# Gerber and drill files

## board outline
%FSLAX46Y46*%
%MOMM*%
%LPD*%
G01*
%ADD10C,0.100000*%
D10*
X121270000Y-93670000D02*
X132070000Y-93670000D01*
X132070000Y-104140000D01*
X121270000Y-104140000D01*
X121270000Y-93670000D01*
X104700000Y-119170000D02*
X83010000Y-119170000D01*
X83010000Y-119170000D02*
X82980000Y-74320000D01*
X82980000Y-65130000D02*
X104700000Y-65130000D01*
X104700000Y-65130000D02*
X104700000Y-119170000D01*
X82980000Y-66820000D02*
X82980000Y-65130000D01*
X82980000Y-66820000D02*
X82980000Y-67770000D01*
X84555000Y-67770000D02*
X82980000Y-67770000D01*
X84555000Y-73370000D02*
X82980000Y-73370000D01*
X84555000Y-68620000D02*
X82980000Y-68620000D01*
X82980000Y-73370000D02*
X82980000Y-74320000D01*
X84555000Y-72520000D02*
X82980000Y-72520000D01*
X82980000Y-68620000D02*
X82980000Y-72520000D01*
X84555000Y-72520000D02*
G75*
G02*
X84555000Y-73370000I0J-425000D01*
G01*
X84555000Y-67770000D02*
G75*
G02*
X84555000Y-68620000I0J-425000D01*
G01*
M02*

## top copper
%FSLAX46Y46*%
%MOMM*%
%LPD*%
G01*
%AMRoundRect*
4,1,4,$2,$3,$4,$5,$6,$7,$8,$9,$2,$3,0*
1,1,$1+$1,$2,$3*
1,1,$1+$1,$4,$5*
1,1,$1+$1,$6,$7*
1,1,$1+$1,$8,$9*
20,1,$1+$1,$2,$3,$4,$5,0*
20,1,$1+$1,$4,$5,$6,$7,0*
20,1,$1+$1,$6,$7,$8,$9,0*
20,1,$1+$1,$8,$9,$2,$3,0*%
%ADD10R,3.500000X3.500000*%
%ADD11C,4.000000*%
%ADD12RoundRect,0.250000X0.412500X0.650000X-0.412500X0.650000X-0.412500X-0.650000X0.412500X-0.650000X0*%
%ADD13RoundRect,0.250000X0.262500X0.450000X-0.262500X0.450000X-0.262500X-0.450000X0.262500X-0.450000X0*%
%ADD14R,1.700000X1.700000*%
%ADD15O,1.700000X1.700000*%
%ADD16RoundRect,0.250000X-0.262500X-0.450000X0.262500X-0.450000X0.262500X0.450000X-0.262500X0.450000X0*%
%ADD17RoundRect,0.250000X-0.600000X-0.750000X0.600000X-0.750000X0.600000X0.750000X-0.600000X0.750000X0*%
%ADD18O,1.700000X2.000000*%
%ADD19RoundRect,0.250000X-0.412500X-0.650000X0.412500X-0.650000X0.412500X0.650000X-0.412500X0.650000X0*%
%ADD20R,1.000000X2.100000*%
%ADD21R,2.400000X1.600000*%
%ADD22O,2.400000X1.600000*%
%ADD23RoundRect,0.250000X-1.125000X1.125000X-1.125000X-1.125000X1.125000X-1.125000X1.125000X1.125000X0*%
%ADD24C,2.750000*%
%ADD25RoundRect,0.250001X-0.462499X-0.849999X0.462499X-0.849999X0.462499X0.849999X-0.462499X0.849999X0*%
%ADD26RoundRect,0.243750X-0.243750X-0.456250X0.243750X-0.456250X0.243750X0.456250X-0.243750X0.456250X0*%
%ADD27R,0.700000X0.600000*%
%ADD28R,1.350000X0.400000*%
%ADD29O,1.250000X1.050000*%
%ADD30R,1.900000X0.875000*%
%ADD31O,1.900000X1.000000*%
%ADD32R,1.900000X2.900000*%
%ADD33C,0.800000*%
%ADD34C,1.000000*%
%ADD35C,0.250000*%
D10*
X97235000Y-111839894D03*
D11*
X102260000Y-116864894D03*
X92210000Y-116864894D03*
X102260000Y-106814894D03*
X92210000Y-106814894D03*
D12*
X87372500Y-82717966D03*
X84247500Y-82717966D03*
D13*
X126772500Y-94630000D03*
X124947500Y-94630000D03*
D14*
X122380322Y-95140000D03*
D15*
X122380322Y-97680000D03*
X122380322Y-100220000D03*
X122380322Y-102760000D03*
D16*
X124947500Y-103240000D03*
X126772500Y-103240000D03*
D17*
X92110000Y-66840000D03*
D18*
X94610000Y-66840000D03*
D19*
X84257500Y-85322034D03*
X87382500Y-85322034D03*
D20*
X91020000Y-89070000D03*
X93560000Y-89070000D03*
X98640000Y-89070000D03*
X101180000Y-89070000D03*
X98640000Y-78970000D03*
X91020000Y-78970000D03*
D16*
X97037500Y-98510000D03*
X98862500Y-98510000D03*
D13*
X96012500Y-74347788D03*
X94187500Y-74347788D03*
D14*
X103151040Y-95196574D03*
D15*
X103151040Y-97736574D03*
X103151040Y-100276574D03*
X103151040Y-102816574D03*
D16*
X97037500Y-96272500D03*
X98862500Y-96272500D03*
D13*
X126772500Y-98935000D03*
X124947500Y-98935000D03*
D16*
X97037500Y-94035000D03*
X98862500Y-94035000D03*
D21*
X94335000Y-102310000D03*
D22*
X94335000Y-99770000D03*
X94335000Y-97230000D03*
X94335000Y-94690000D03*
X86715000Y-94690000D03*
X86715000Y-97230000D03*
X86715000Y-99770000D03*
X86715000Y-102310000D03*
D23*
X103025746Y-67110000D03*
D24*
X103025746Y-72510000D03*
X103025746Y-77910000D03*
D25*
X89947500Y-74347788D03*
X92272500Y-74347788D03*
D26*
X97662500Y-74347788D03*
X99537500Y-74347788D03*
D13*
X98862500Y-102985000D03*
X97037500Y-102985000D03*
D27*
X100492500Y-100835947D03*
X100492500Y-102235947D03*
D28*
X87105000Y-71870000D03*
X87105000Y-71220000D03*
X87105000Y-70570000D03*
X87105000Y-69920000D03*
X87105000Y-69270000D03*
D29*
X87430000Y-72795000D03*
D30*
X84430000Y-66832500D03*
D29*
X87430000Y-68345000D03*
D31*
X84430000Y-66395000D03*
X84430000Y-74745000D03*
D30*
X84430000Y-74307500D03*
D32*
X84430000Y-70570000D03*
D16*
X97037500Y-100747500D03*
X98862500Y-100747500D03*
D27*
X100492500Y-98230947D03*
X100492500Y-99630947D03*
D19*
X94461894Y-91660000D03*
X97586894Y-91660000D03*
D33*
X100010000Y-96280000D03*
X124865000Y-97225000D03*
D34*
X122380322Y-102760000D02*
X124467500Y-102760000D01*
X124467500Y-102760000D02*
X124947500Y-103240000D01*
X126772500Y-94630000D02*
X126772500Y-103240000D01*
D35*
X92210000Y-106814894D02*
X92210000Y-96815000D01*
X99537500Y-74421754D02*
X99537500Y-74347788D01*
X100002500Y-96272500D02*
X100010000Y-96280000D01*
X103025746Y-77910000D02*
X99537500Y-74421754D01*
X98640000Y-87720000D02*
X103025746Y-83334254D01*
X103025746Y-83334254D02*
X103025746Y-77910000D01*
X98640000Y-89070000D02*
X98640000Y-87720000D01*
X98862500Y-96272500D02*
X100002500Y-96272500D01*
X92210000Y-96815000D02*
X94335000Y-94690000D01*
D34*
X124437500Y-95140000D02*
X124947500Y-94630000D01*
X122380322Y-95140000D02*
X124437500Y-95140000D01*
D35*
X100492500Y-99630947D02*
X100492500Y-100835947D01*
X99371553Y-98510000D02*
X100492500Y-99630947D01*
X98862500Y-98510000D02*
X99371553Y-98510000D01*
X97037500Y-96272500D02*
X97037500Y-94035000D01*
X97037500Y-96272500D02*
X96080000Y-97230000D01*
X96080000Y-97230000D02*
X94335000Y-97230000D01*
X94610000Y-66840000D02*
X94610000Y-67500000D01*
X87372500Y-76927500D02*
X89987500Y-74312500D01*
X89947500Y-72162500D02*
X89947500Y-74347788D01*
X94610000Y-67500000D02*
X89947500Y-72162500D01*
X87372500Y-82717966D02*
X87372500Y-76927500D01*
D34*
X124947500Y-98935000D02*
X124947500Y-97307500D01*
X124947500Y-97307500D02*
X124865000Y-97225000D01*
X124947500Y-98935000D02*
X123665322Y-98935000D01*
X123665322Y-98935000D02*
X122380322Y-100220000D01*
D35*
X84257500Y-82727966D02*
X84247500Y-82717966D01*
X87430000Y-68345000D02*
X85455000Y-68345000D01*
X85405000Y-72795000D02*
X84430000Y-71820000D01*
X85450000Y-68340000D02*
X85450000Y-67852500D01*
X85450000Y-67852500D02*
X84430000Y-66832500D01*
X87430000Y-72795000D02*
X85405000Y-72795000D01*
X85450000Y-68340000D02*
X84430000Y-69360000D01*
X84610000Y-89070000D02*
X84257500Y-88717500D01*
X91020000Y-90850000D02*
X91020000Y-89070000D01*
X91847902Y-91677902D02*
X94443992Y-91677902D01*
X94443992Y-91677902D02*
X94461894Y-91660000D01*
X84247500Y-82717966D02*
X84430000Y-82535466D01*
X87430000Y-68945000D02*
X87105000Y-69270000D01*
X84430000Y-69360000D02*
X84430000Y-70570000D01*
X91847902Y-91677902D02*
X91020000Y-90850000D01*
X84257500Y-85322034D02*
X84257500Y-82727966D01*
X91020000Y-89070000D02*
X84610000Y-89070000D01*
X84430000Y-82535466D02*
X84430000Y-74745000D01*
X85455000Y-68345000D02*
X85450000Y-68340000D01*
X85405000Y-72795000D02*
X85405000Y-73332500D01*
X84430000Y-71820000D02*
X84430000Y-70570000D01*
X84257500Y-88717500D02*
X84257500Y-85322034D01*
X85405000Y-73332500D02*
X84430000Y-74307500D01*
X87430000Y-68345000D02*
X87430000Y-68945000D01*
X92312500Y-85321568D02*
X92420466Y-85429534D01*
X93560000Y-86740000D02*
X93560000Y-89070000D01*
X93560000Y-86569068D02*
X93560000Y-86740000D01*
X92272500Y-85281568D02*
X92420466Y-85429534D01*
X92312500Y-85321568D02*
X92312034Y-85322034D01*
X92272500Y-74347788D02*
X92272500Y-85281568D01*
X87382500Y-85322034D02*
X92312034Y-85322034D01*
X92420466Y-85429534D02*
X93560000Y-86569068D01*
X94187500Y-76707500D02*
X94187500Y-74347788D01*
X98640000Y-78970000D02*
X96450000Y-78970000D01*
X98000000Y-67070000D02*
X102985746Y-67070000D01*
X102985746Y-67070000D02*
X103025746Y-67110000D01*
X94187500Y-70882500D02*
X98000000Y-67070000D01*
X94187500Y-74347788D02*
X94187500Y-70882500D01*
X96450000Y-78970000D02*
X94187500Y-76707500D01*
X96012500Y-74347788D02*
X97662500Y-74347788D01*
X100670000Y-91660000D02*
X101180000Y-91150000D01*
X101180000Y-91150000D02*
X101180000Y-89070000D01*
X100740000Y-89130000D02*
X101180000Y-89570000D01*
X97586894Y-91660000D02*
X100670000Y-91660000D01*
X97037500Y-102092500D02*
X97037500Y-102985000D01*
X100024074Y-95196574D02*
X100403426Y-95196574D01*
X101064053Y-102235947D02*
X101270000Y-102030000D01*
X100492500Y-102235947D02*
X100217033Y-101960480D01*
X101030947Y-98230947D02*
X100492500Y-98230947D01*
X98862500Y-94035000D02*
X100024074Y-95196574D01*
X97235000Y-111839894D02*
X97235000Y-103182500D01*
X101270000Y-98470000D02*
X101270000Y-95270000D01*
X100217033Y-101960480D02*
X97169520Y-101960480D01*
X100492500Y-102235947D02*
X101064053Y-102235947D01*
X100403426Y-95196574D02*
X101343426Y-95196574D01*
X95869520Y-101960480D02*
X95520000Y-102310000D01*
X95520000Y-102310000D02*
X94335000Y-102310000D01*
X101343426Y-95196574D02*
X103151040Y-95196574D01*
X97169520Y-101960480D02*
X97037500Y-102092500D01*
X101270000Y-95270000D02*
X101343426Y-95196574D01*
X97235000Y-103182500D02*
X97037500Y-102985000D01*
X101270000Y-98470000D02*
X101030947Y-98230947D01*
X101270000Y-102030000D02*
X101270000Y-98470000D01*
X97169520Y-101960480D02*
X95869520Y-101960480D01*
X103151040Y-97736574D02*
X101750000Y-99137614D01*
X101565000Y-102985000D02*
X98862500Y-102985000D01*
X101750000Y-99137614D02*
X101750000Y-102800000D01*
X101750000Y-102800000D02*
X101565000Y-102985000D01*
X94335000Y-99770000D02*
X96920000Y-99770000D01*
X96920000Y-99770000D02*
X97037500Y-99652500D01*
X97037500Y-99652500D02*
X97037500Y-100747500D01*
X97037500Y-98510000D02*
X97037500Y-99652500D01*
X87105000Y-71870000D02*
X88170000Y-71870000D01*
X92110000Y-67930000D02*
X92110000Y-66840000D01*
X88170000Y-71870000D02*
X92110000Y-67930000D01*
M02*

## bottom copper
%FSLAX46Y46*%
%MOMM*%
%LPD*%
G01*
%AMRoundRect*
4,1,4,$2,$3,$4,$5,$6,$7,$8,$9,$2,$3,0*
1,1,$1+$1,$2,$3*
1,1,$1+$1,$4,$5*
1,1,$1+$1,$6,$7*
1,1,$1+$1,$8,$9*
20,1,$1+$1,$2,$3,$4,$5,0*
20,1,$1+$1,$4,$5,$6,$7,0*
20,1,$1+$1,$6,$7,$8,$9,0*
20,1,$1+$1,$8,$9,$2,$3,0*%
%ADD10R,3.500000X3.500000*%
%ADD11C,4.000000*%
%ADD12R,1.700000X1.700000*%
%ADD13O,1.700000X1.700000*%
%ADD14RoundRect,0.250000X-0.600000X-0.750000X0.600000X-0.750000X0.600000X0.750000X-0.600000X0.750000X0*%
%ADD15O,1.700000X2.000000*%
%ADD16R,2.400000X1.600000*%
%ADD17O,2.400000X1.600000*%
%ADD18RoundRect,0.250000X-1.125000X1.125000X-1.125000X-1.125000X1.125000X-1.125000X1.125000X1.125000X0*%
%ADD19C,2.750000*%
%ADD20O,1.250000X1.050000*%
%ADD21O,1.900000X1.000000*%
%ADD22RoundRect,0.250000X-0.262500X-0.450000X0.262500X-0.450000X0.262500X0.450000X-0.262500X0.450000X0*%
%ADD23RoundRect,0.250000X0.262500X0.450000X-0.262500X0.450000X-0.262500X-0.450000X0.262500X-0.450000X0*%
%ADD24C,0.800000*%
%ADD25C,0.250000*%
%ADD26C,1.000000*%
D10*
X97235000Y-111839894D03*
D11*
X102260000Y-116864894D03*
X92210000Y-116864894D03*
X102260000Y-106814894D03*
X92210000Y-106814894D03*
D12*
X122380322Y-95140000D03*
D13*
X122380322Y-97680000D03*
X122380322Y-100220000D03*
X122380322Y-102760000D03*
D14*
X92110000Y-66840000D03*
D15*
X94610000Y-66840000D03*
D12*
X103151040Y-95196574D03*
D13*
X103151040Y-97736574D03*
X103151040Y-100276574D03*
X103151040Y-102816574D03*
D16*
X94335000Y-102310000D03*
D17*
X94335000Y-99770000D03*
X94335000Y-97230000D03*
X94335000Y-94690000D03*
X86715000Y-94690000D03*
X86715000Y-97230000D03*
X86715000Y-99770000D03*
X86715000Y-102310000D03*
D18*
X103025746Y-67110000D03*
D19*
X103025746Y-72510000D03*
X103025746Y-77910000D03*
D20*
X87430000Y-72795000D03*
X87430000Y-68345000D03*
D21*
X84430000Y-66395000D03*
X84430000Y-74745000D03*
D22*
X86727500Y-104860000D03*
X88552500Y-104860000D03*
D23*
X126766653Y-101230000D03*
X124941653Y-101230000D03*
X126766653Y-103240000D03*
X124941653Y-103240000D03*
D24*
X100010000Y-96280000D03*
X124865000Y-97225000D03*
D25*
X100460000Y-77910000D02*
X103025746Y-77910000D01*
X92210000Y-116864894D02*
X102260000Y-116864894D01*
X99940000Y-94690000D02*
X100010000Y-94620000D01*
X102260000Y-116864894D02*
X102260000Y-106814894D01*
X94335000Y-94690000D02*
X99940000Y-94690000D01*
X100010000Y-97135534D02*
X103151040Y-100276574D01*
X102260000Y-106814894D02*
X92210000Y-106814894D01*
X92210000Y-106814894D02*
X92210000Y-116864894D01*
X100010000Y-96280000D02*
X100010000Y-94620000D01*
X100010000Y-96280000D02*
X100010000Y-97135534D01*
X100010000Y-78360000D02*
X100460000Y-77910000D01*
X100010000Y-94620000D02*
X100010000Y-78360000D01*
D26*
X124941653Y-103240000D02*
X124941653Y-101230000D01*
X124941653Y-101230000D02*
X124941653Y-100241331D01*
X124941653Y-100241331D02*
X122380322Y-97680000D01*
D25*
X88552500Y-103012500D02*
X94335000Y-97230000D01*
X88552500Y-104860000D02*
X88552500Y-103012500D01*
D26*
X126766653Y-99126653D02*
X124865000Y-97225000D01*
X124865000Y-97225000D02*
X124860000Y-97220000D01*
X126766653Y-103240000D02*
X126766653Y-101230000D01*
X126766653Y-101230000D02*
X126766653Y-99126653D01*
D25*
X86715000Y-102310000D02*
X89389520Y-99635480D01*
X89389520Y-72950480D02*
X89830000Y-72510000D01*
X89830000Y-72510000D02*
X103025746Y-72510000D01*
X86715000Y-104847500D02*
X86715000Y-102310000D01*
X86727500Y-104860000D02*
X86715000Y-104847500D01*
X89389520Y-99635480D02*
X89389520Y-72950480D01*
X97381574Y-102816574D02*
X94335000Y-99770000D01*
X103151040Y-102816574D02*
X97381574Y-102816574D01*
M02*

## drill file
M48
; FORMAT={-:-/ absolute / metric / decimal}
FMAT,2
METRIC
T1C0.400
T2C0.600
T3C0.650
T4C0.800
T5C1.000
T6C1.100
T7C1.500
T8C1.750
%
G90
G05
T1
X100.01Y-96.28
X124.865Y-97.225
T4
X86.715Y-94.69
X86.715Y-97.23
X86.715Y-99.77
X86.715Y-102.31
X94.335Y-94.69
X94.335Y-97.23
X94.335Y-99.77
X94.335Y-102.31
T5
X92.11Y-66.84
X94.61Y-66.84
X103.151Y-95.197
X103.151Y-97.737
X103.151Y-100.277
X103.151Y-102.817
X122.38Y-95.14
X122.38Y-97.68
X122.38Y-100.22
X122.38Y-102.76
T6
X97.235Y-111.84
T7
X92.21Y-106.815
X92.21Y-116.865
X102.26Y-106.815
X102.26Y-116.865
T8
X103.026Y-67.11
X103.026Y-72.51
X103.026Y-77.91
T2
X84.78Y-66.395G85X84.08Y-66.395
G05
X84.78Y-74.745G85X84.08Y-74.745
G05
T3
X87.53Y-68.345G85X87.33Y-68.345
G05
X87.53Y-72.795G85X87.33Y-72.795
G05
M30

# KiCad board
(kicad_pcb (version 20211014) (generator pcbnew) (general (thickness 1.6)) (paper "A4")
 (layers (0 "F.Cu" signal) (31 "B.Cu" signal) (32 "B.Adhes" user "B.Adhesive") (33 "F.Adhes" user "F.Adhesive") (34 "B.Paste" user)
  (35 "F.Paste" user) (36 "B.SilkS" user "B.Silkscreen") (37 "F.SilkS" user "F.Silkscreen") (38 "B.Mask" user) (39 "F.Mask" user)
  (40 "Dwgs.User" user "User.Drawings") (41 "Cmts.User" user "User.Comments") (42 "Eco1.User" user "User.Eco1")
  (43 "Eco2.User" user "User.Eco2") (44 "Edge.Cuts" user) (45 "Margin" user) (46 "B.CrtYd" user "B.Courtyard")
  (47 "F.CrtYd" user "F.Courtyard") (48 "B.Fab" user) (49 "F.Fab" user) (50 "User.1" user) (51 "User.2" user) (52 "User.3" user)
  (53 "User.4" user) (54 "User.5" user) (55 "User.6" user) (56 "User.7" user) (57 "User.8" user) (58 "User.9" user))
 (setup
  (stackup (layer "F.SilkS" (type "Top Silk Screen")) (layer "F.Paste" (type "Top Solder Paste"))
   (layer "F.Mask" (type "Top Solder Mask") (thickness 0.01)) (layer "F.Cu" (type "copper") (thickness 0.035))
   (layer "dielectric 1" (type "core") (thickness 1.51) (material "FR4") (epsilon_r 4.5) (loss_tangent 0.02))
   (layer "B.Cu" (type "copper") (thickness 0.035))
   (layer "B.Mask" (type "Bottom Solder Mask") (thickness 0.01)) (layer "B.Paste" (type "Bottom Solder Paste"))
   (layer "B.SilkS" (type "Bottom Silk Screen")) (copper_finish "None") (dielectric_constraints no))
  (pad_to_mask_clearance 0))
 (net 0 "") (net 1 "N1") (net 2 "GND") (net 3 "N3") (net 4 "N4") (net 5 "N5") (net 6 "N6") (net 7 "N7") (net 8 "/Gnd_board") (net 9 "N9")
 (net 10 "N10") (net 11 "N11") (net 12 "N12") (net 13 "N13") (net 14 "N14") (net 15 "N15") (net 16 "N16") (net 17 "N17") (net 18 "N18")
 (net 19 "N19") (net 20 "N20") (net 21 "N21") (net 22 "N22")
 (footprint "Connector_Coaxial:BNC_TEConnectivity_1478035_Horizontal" (layer "F.Cu") (at 97.235 111.839894 -90)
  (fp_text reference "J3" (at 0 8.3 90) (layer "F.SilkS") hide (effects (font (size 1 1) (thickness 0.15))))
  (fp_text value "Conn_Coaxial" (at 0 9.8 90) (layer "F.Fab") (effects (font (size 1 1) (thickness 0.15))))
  (pad "1" thru_hole rect (at 0 0 270) (size 3.5 3.5) (drill 1.1) (layers *.Cu *.Mask) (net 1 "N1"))
  (pad "2" thru_hole circle (at 5.025 -5.025 270) (size 4 4) (drill 1.5) (layers *.Cu *.Mask) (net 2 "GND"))
  (pad "2" thru_hole circle (at 5.025 5.025 270) (size 4 4) (drill 1.5) (layers *.Cu *.Mask) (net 2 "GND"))
  (pad "2" thru_hole circle (at -5.025 -5.025 270) (size 4 4) (drill 1.5) (layers *.Cu *.Mask) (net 2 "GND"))
  (pad "2" thru_hole circle (at -5.025 5.025 270) (size 4 4) (drill 1.5) (layers *.Cu *.Mask) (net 2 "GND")))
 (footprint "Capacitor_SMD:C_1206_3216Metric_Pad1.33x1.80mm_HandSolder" (layer "F.Cu") (at 85.81 82.717966 180)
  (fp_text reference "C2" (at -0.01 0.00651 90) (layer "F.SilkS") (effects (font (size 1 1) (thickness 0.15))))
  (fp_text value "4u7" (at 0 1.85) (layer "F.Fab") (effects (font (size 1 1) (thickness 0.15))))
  (pad "1" smd roundrect locked (at -1.5625 0 180) (size 1.325 1.8) (layers "F.Cu" "F.Paste" "F.Mask") (roundrect_rratio 0.188679)
   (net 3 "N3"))
  (pad "2" smd roundrect locked (at 1.5625 0 180) (size 1.325 1.8) (layers "F.Cu" "F.Paste" "F.Mask") (roundrect_rratio 0.188679)
   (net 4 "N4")))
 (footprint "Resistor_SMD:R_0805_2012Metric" (layer "F.Cu") (at 125.86 94.63 180)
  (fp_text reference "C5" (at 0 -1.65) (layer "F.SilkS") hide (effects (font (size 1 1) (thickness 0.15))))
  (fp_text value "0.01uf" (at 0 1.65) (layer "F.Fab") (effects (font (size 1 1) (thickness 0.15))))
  (pad "1" smd roundrect locked (at -0.9125 0 180) (size 1.025 1.4) (layers "F.Cu" "F.Paste" "F.Mask") (roundrect_rratio 0.243902)
   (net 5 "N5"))
  (pad "2" smd roundrect locked (at 0.9125 0 180) (size 1.025 1.4) (layers "F.Cu" "F.Paste" "F.Mask") (roundrect_rratio 0.243902)
   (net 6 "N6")))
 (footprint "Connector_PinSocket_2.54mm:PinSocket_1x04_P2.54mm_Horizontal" (layer "F.Cu") (at 122.380322 95.14)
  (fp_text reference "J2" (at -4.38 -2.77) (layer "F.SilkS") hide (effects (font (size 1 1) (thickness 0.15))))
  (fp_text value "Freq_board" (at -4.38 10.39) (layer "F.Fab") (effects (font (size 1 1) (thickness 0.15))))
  (pad "1" thru_hole rect locked (at 0 0) (size 1.7 1.7) (drill 1) (layers *.Cu *.Mask) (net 6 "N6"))
  (pad "2" thru_hole oval locked (at 0 2.54) (size 1.7 1.7) (drill 1) (layers *.Cu *.Mask) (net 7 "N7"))
  (pad "3" thru_hole oval locked (at 0 5.08) (size 1.7 1.7) (drill 1) (layers *.Cu *.Mask) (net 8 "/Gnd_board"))
  (pad "4" thru_hole oval locked (at 0 7.62) (size 1.7 1.7) (drill 1) (layers *.Cu *.Mask) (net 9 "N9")))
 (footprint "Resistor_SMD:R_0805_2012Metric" (layer "F.Cu") (at 125.86 103.24)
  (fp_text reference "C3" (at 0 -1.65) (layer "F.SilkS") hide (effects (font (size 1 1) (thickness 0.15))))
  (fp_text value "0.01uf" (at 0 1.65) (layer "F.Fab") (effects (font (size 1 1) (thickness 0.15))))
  (pad "1" smd roundrect locked (at -0.9125 0) (size 1.025 1.4) (layers "F.Cu" "F.Paste" "F.Mask") (roundrect_rratio 0.243902) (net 9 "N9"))
  (pad "2" smd roundrect locked (at 0.9125 0) (size 1.025 1.4) (layers "F.Cu" "F.Paste" "F.Mask") (roundrect_rratio 0.243902) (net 5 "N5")))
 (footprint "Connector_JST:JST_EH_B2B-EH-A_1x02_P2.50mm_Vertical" (layer "F.Cu") (at 92.11 66.84)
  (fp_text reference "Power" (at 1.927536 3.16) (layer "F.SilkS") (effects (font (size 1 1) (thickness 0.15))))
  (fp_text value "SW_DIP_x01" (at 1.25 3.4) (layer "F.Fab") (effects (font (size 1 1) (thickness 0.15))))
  (pad "1" thru_hole roundrect locked (at 0 0) (size 1.7 2) (drill 1) (layers *.Cu *.Mask) (roundrect_rratio 0.147059) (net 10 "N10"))
  (pad "2" thru_hole oval locked (at 2.5 0) (size 1.7 2) (drill 1) (layers *.Cu *.Mask) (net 3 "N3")))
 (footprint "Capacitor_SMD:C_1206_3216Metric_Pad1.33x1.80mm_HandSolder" (layer "F.Cu") (at 85.82 85.322034)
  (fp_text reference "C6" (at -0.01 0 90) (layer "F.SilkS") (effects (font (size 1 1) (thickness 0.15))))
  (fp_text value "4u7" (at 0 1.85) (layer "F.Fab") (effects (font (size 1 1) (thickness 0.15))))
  (pad "1" smd roundrect locked (at -1.5625 0) (size 1.325 1.8) (layers "F.Cu" "F.Paste" "F.Mask") (roundrect_rratio 0.188679) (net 4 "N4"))
  (pad "2" smd roundrect locked (at 1.5625 0) (size 1.325 1.8) (layers "F.Cu" "F.Paste" "F.Mask") (roundrect_rratio 0.188679) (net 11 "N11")))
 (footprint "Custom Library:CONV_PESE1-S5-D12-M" (layer "F.Cu") (at 96.1 84.02 90)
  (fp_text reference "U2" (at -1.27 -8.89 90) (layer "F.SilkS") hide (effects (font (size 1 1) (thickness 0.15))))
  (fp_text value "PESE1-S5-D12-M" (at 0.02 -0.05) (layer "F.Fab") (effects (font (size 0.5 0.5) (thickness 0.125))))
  (pad "1" smd rect (at -5.05 -5.08 90) (size 2.1 1) (layers "F.Cu" "F.Paste" "F.Mask") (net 4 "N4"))
  (pad "2" smd rect (at -5.05 -2.54 90) (size 2.1 1) (layers "F.Cu" "F.Paste" "F.Mask") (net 11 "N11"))
  (pad "4" smd rect (at -5.05 2.54 90) (size 2.1 1) (layers "F.Cu" "F.Paste" "F.Mask") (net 2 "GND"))
  (pad "5" smd rect (at -5.05 5.08 90) (size 2.1 1) (layers "F.Cu" "F.Paste" "F.Mask") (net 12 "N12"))
  (pad "7" smd rect (at 5.05 2.54 90) (size 2.1 1) (layers "F.Cu" "F.Paste" "F.Mask") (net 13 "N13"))
  (pad "10" smd rect (at 5.05 -5.08 90) (size 2.1 1) (layers "F.Cu" "F.Paste" "F.Mask")))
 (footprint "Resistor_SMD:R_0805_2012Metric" (layer "F.Cu") (at 97.95 98.51)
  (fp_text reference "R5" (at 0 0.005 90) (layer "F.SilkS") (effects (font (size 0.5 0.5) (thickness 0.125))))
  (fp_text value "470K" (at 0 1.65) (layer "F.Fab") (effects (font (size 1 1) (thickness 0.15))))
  (pad "1" smd roundrect locked (at -0.9125 0) (size 1.025 1.4) (layers "F.Cu" "F.Paste" "F.Mask") (roundrect_rratio 0.243902)
   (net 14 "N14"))
  (pad "2" smd roundrect locked (at 0.9125 0) (size 1.025 1.4) (layers "F.Cu" "F.Paste" "F.Mask") (roundrect_rratio 0.243902) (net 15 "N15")))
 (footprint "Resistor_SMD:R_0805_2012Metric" (layer "F.Cu") (at 95.1 74.347788 180)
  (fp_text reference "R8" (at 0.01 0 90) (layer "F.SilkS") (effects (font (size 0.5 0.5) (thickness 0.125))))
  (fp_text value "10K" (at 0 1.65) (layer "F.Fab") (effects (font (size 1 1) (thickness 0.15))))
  (pad "1" smd roundrect locked (at -0.9125 0 180) (size 1.025 1.4) (layers "F.Cu" "F.Paste" "F.Mask") (roundrect_rratio 0.243902)
   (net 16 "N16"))
  (pad "2" smd roundrect locked (at 0.9125 0 180) (size 1.025 1.4) (layers "F.Cu" "F.Paste" "F.Mask") (roundrect_rratio 0.243902)
   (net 13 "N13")))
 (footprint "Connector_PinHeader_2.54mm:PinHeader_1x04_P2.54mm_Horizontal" (layer "F.Cu") (at 103.15104 95.196574)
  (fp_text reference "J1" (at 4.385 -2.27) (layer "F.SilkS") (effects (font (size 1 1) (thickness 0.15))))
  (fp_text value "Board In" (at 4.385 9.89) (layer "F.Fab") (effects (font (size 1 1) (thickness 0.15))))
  (pad "1" thru_hole rect locked (at 0 0) (size 1.7 1.7) (drill 1) (layers *.Cu *.Mask) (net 1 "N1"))
  (pad "2" thru_hole oval locked (at 0 2.54) (size 1.7 1.7) (drill 1) (layers *.Cu *.Mask) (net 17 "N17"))
  (pad "3" thru_hole oval locked (at 0 5.08) (size 1.7 1.7) (drill 1) (layers *.Cu *.Mask) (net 2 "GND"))
  (pad "4" thru_hole oval locked (at 0 7.62) (size 1.7 1.7) (drill 1) (layers *.Cu *.Mask) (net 14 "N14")))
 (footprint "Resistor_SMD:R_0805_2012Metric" (layer "F.Cu") (at 97.95 96.2725)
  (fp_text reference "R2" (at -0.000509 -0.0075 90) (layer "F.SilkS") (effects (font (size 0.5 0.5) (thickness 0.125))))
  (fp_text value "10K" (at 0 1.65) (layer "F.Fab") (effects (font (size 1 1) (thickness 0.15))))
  (pad "1" smd roundrect locked (at -0.9125 0) (size 1.025 1.4) (layers "F.Cu" "F.Paste" "F.Mask") (roundrect_rratio 0.243902)
   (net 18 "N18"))
  (pad "2" smd roundrect locked (at 0.9125 0) (size 1.025 1.4) (layers "F.Cu" "F.Paste" "F.Mask") (roundrect_rratio 0.243902) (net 2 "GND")))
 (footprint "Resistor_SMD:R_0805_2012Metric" (layer "F.Cu") (at 125.86 98.935 180)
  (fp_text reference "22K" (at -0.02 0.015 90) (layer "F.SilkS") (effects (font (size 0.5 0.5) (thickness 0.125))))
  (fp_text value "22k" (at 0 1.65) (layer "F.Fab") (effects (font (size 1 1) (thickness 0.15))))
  (pad "1" smd roundrect locked (at -0.9125 0 180) (size 1.025 1.4) (layers "F.Cu" "F.Paste" "F.Mask") (roundrect_rratio 0.243902)
   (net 5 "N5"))
  (pad "2" smd roundrect locked (at 0.9125 0 180) (size 1.025 1.4) (layers "F.Cu" "F.Paste" "F.Mask") (roundrect_rratio 0.243902)
   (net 8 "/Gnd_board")))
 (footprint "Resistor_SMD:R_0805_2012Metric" (layer "F.Cu") (at 97.95 94.035)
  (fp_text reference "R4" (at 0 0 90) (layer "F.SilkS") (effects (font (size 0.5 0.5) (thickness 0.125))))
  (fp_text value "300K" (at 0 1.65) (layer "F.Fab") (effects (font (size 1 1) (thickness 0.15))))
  (pad "1" smd roundrect locked (at -0.9125 0) (size 1.025 1.4) (layers "F.Cu" "F.Paste" "F.Mask") (roundrect_rratio 0.243902)
   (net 18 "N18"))
  (pad "2" smd roundrect locked (at 0.9125 0) (size 1.025 1.4) (layers "F.Cu" "F.Paste" "F.Mask") (roundrect_rratio 0.243902) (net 1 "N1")))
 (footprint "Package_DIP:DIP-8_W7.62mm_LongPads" (layer "F.Cu") (at 94.335 102.31 180)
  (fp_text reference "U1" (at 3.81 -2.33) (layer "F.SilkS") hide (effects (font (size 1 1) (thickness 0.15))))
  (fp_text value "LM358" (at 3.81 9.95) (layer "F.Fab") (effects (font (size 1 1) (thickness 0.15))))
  (pad "1" thru_hole rect locked (at 0 0 180) (size 2.4 1.6) (drill 0.8) (layers *.Cu *.Mask) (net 1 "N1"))
  (pad "2" thru_hole oval locked (at 0 2.54 180) (size 2.4 1.6) (drill 0.8) (layers *.Cu *.Mask) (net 14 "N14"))
  (pad "3" thru_hole oval locked (at 0 5.08 180) (size 2.4 1.6) (drill 0.8) (layers *.Cu *.Mask) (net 18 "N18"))
  (pad "4" thru_hole oval locked (at 0 7.62 180) (size 2.4 1.6) (drill 0.8) (layers *.Cu *.Mask) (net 2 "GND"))
  (pad "5" thru_hole oval locked (at 7.62 7.62 180) (size 2.4 1.6) (drill 0.8) (layers *.Cu *.Mask))
  (pad "6" thru_hole oval locked (at 7.62 5.08 180) (size 2.4 1.6) (drill 0.8) (layers *.Cu *.Mask))
  (pad "7" thru_hole oval locked (at 7.62 2.54 180) (size 2.4 1.6) (drill 0.8) (layers *.Cu *.Mask))
  (pad "8" thru_hole oval locked (at 7.62 0 180) (size 2.4 1.6) (drill 0.8) (layers *.Cu *.Mask) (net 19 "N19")))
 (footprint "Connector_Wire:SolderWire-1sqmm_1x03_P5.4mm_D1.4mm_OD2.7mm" (layer "F.Cu") (at 103.025746 67.11 -90)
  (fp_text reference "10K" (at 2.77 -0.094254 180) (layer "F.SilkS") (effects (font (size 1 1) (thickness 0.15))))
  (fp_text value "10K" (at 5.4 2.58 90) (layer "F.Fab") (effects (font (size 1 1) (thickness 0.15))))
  (pad "1" thru_hole roundrect locked (at 0 0 270) (size 2.75 2.75) (drill 1.75) (layers *.Cu *.Mask) (roundrect_rratio 0.090909)
   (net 13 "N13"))
  (pad "2" thru_hole circle locked (at 5.4 0 270) (size 2.75 2.75) (drill 1.75) (layers *.Cu *.Mask) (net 19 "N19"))
  (pad "3" thru_hole circle locked (at 10.8 0 270) (size 2.75 2.75) (drill 1.75) (layers *.Cu *.Mask) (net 2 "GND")))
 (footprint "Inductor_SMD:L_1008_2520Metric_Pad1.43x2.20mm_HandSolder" (layer "F.Cu") (at 91.11 74.347788)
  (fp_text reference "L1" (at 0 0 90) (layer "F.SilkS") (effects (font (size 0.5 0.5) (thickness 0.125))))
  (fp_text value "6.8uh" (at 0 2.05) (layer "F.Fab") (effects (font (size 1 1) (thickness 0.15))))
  (pad "1" smd roundrect locked (at -1.1625 0) (size 1.425 2.2) (layers "F.Cu" "F.Paste" "F.Mask") (roundrect_rratio 0.175439) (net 3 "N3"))
  (pad "2" smd roundrect locked (at 1.1625 0) (size 1.425 2.2) (layers "F.Cu" "F.Paste" "F.Mask") (roundrect_rratio 0.175439) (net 11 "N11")))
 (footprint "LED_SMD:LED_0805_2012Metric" (layer "F.Cu") (at 98.6 74.347788)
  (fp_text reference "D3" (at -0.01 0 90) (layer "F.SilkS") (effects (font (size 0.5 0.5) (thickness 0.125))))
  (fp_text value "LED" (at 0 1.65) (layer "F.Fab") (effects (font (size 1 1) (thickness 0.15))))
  (pad "1" smd roundrect locked (at -0.9375 0) (size 0.975 1.4) (layers "F.Cu" "F.Paste" "F.Mask") (roundrect_rratio 0.25) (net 16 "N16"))
  (pad "2" smd roundrect locked (at 0.9375 0) (size 0.975 1.4) (layers "F.Cu" "F.Paste" "F.Mask") (roundrect_rratio 0.25) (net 2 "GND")))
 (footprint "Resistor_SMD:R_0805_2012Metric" (layer "F.Cu") (at 97.95 102.985 180)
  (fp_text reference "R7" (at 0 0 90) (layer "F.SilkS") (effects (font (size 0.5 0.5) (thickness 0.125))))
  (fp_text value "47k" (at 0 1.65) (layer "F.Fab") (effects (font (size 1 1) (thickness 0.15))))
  (pad "1" smd roundrect locked (at -0.9125 0 180) (size 1.025 1.4) (layers "F.Cu" "F.Paste" "F.Mask") (roundrect_rratio 0.243902)
   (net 17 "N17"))
  (pad "2" smd roundrect locked (at 0.9125 0 180) (size 1.025 1.4) (layers "F.Cu" "F.Paste" "F.Mask") (roundrect_rratio 0.243902)
   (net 1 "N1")))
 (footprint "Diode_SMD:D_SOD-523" (layer "F.Cu") (at 100.4925 101.535947 -90)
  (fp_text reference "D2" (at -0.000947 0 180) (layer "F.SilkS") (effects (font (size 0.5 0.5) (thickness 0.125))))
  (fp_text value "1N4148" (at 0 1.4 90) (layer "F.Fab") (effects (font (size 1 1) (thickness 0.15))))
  (pad "1" smd rect locked (at -0.7 0 90) (size 0.6 0.7) (layers "F.Cu" "F.Paste" "F.Mask") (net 15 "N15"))
  (pad "2" smd rect locked (at 0.7 0 90) (size 0.6 0.7) (layers "F.Cu" "F.Paste" "F.Mask") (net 1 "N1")))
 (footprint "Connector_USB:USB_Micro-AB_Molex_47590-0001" (layer "F.Cu") (at 84.43 70.57 -90)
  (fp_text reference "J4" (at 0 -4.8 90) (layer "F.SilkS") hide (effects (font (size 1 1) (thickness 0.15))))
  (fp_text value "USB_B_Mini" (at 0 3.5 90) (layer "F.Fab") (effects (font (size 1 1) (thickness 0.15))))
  (fp_line (start -3.75 1.45) (end -2.8 1.45) (layer "Edge.Cuts") (width 0.1))
  (fp_line (start -2.8 -0.125) (end -2.8 1.45) (layer "Edge.Cuts") (width 0.1))
  (fp_line (start 2.8 -0.125) (end 2.8 1.45) (layer "Edge.Cuts") (width 0.1))
  (fp_line (start -1.95 -0.125) (end -1.95 1.45) (layer "Edge.Cuts") (width 0.1))
  (fp_line (start 2.8 1.45) (end 3.75 1.45) (layer "Edge.Cuts") (width 0.1))
  (fp_line (start 1.95 -0.125) (end 1.95 1.45) (layer "Edge.Cuts") (width 0.1))
  (fp_line (start -1.95 1.45) (end 1.95 1.45) (layer "Edge.Cuts") (width 0.1))
  (fp_arc (start 1.95 -0.125) (mid 2.375 -0.55) (end 2.8 -0.125) (layer "Edge.Cuts") (width 0.1))
  (fp_arc (start -2.8 -0.125) (mid -2.375 -0.55) (end -1.95 -0.125) (layer "Edge.Cuts") (width 0.1))
  (pad "" smd rect locked (at -3.5 0 270) (size 0.3 0.85) (layers "F.Paste"))
  (pad "" smd rect locked (at 3.5 0 270) (size 0.3 0.85) (layers "F.Paste"))
  (pad "1" smd rect locked (at 1.3 -2.675 270) (size 0.4 1.35) (layers "F.Cu" "F.Paste" "F.Mask") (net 10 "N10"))
  (pad "2" smd rect locked (at 0.65 -2.675 270) (size 0.4 1.35) (layers "F.Cu" "F.Paste" "F.Mask") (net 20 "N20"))
  (pad "3" smd rect locked (at 0 -2.675 270) (size 0.4 1.35) (layers "F.Cu" "F.Paste" "F.Mask") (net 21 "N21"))
  (pad "4" smd rect locked (at -0.65 -2.675 270) (size 0.4 1.35) (layers "F.Cu" "F.Paste" "F.Mask") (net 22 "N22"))
  (pad "5" smd rect locked (at -1.3 -2.675 270) (size 0.4 1.35) (layers "F.Cu" "F.Paste" "F.Mask") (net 4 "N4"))
  (pad "6" thru_hole oval locked (at 2.225 -3 270) (size 1.05 1.25) (drill oval 0.65 0.85) (layers *.Cu *.Mask) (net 4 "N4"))
  (pad "6" smd rect locked (at -3.7375 0 270) (size 0.875 1.9) (layers "F.Cu" "F.Mask") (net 4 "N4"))
  (pad "6" thru_hole oval locked (at -2.225 -3 270) (size 1.05 1.25) (drill oval 0.65 0.85) (layers *.Cu *.Mask) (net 4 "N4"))
  (pad "6" thru_hole oval locked (at -4.175 0 270) (size 1 1.9) (drill oval 0.6 1.3) (layers *.Cu *.Mask) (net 4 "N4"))
  (pad "6" thru_hole oval locked (at 4.175 0 270) (size 1 1.9) (drill oval 0.6 1.3) (layers *.Cu *.Mask) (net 4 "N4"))
  (pad "6" smd rect locked (at 3.7375 0 270) (size 0.875 1.9) (layers "F.Cu" "F.Mask") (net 4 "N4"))
  (pad "6" smd rect locked (at 0 0 270) (size 2.9 1.9) (layers "F.Cu" "F.Paste" "F.Mask") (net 4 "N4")))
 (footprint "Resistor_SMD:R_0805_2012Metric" (layer "F.Cu") (at 97.95 100.7475)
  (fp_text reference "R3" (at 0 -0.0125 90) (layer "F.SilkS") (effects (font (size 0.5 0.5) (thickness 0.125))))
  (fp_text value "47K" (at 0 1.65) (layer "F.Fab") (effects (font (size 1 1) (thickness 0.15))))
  (pad "1" smd roundrect locked (at -0.9125 0) (size 1.025 1.4) (layers "F.Cu" "F.Paste" "F.Mask") (roundrect_rratio 0.243902)
   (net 14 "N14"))
  (pad "2" smd roundrect locked (at 0.9125 0) (size 1.025 1.4) (layers "F.Cu" "F.Paste" "F.Mask") (roundrect_rratio 0.243902) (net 17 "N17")))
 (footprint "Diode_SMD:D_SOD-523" (layer "F.Cu") (at 100.4925 98.930947 -90)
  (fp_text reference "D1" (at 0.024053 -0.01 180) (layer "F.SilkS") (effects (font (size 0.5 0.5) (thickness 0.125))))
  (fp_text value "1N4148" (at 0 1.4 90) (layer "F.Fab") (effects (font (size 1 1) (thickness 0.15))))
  (pad "1" smd rect locked (at -0.7 0 90) (size 0.6 0.7) (layers "F.Cu" "F.Paste" "F.Mask") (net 1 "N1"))
  (pad "2" smd rect locked (at 0.7 0 90) (size 0.6 0.7) (layers "F.Cu" "F.Paste" "F.Mask") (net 15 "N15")))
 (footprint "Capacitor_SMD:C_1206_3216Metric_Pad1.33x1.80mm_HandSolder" (layer "F.Cu") (at 96.024394 91.66)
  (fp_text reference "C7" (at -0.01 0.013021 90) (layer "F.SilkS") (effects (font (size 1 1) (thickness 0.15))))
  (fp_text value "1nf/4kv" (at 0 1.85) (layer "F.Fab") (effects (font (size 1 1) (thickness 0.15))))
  (pad "1" smd roundrect locked (at -1.5625 0) (size 1.325 1.8) (layers "F.Cu" "F.Paste" "F.Mask") (roundrect_rratio 0.188679) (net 4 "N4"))
  (pad "2" smd roundrect locked (at 1.5625 0) (size 1.325 1.8) (layers "F.Cu" "F.Paste" "F.Mask") (roundrect_rratio 0.188679) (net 12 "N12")))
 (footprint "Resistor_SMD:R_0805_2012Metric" (layer "B.Cu") (at 87.64 104.86)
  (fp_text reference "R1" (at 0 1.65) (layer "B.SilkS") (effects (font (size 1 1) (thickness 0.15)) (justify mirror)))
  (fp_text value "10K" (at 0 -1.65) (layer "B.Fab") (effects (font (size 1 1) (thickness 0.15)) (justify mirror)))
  (pad "1" smd roundrect locked (at -0.9125 0) (size 1.025 1.4) (layers "B.Cu" "B.Paste" "B.Mask") (roundrect_rratio 0.243902)
   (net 19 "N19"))
  (pad "2" smd roundrect locked (at 0.9125 0) (size 1.025 1.4) (layers "B.Cu" "B.Paste" "B.Mask") (roundrect_rratio 0.243902) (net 18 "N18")))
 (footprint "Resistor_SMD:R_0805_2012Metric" (layer "B.Cu") (at 125.854153 101.23 180)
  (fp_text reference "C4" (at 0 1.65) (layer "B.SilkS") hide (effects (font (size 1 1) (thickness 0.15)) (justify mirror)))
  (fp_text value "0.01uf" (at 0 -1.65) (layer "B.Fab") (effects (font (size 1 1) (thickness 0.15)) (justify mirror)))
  (pad "1" smd roundrect locked (at -0.9125 0 180) (size 1.025 1.4) (layers "B.Cu" "B.Paste" "B.Mask") (roundrect_rratio 0.243902)
   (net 8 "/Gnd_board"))
  (pad "2" smd roundrect locked (at 0.9125 0 180) (size 1.025 1.4) (layers "B.Cu" "B.Paste" "B.Mask") (roundrect_rratio 0.243902)
   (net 7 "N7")))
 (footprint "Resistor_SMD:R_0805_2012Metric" (layer "B.Cu") (at 125.854153 103.24 180)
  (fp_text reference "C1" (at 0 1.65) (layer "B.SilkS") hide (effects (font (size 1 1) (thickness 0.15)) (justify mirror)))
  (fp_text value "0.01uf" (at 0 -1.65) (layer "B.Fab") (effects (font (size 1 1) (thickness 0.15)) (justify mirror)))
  (pad "1" smd roundrect locked (at -0.9125 0 180) (size 1.025 1.4) (layers "B.Cu" "B.Paste" "B.Mask") (roundrect_rratio 0.243902)
   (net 8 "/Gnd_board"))
  (pad "2" smd roundrect locked (at 0.9125 0 180) (size 1.025 1.4) (layers "B.Cu" "B.Paste" "B.Mask") (roundrect_rratio 0.243902)
   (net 7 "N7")))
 (gr_rect (start 121.27 93.67) (end 132.07 104.14) (layer "Edge.Cuts") (width 0.1) (fill none))
 (gr_line (start 104.7 119.17) (end 83.01 119.17) (layer "Edge.Cuts") (width 0.1))
 (gr_line (start 83.01 119.17) (end 82.98 74.32) (layer "Edge.Cuts") (width 0.1))
 (gr_line (start 82.98 65.13) (end 104.7 65.13) (layer "Edge.Cuts") (width 0.1))
 (gr_line (start 104.7 65.13) (end 104.7 119.17) (layer "Edge.Cuts") (width 0.1))
 (gr_line (start 82.98 66.82) (end 82.98 65.13) (layer "Edge.Cuts") (width 0.1))
 (segment (start 122.380322 102.76) (end 124.4675 102.76) (width 1) (layer "F.Cu") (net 9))
 (segment (start 124.4675 102.76) (end 124.9475 103.24) (width 1) (layer "F.Cu") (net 9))
 (segment (start 126.7725 94.63) (end 126.7725 103.24) (width 1) (layer "F.Cu") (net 5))
 (segment (start 92.21 106.814894) (end 92.21 96.815) (width 0.25) (layer "F.Cu") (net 2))
 (segment (start 99.5375 74.421754) (end 99.5375 74.347788) (width 0.25) (layer "F.Cu") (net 2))
 (segment (start 100.0025 96.2725) (end 100.01 96.28) (width 0.25) (layer "F.Cu") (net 2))
 (segment (start 103.025746 77.91) (end 99.5375 74.421754) (width 0.25) (layer "F.Cu") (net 2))
 (segment (start 98.64 87.72) (end 103.025746 83.334254) (width 0.25) (layer "F.Cu") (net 2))
 (segment (start 103.025746 83.334254) (end 103.025746 77.91) (width 0.25) (layer "F.Cu") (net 2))
 (segment (start 98.64 89.07) (end 98.64 87.72) (width 0.25) (layer "F.Cu") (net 2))
 (segment (start 98.8625 96.2725) (end 100.0025 96.2725) (width 0.25) (layer "F.Cu") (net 2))
 (segment (start 92.21 96.815) (end 94.335 94.69) (width 0.25) (layer "F.Cu") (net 2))
 (via (at 100.01 96.28) (size 0.8) (drill 0.4) (layers "F.Cu" "B.Cu") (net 2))
 (segment (start 100.46 77.91) (end 103.025746 77.91) (width 0.25) (layer "B.Cu") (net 2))
 (segment (start 92.21 116.864894) (end 102.26 116.864894) (width 0.25) (layer "B.Cu") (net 2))
 (segment (start 99.94 94.69) (end 100.01 94.62) (width 0.25) (layer "B.Cu") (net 2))
 (segment (start 102.26 116.864894) (end 102.26 106.814894) (width 0.25) (layer "B.Cu") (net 2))
 (segment (start 94.335 94.69) (end 99.94 94.69) (width 0.25) (layer "B.Cu") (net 2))
 (segment (start 100.01 97.135534) (end 103.15104 100.276574) (width 0.25) (layer "B.Cu") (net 2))
 (segment (start 102.26 106.814894) (end 92.21 106.814894) (width 0.25) (layer "B.Cu") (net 2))
 (segment (start 92.21 106.814894) (end 92.21 116.864894) (width 0.25) (layer "B.Cu") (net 2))
 (segment (start 100.01 96.28) (end 100.01 94.62) (width 0.25) (layer "B.Cu") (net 2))
 (segment (start 100.01 96.28) (end 100.01 97.135534) (width 0.25) (layer "B.Cu") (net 2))
 (segment (start 100.01 78.36) (end 100.46 77.91) (width 0.25) (layer "B.Cu") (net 2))
 (segment (start 100.01 94.62) (end 100.01 78.36) (width 0.25) (layer "B.Cu") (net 2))
 (segment (start 124.941653 103.24) (end 124.941653 101.23) (width 1) (layer "B.Cu") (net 7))
 (segment (start 124.941653 101.23) (end 124.941653 100.241331) (width 1) (layer "B.Cu") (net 7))
 (segment (start 124.941653 100.241331) (end 122.380322 97.68) (width 1) (layer "B.Cu") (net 7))
 (segment (start 124.4375 95.14) (end 124.9475 94.63) (width 1) (layer "F.Cu") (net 6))
 (segment (start 122.380322 95.14) (end 124.4375 95.14) (width 1) (layer "F.Cu") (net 6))
 (segment (start 100.4925 99.630947) (end 100.4925 100.835947) (width 0.25) (layer "F.Cu") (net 15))
 (segment (start 99.371553 98.51) (end 100.4925 99.630947) (width 0.25) (layer "F.Cu") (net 15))
 (segment (start 98.8625 98.51) (end 99.371553 98.51) (width 0.25) (layer "F.Cu") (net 15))
 (segment (start 97.0375 96.2725) (end 97.0375 94.035) (width 0.25) (layer "F.Cu") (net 18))
 (segment (start 97.0375 96.2725) (end 96.08 97.23) (width 0.25) (layer "F.Cu") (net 18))
 (segment (start 96.08 97.23) (end 94.335 97.23) (width 0.25) (layer "F.Cu") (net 18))
 (segment (start 88.5525 103.0125) (end 94.335 97.23) (width 0.25) (layer "B.Cu") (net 18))
 (segment (start 88.5525 104.86) (end 88.5525 103.0125) (width 0.25) (layer "B.Cu") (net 18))
 (segment (start 94.61 66.84) (end 94.61 67.5) (width 0.25) (layer "F.Cu") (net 3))
 (segment (start 87.3725 76.9275) (end 89.9875 74.3125) (width 0.25) (layer "F.Cu") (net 3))
 (segment (start 89.9475 72.1625) (end 89.9475 74.347788) (width 0.25) (layer "F.Cu") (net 3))
 (segment (start 94.61 67.5) (end 89.9475 72.1625) (width 0.25) (layer "F.Cu") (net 3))
 (segment (start 87.3725 82.717966) (end 87.3725 76.9275) (width 0.25) (layer "F.Cu") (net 3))
 (segment (start 124.9475 98.935) (end 124.9475 97.3075) (width 1) (layer "F.Cu") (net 8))
 (segment (start 124.9475 97.3075) (end 124.865 97.225) (width 1) (layer "F.Cu") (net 8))
 (segment (start 124.9475 98.935) (end 123.665322 98.935) (width 1) (layer "F.Cu") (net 8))
 (segment (start 123.665322 98.935) (end 122.380322 100.22) (width 1) (layer "F.Cu") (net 8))
 (via (at 124.865 97.225) (size 0.8) (drill 0.4) (layers "F.Cu" "B.Cu") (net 8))
 (segment (start 126.766653 99.126653) (end 124.865 97.225) (width 1) (layer "B.Cu") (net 8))
 (segment (start 124.865 97.225) (end 124.86 97.22) (width 1) (layer "B.Cu") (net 8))
 (segment (start 126.766653 103.24) (end 126.766653 101.23) (width 1) (layer "B.Cu") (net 8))
 (segment (start 126.766653 101.23) (end 126.766653 99.126653) (width 1) (layer "B.Cu") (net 8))
 (segment (start 84.2575 82.727966) (end 84.2475 82.717966) (width 0.25) (layer "F.Cu") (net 4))
 (segment (start 87.43 68.345) (end 85.455 68.345) (width 0.25) (layer "F.Cu") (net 4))
 (segment (start 85.405 72.795) (end 84.43 71.82) (width 0.25) (layer "F.Cu") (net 4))
 (segment (start 85.45 68.34) (end 85.45 67.8525) (width 0.25) (layer "F.Cu") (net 4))
 (segment (start 85.45 67.8525) (end 84.43 66.8325) (width 0.25) (layer "F.Cu") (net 4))
 (segment (start 87.43 72.795) (end 85.405 72.795) (width 0.25) (layer "F.Cu") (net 4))
 (segment (start 85.45 68.34) (end 84.43 69.36) (width 0.25) (layer "F.Cu") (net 4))
 (segment (start 84.61 89.07) (end 84.2575 88.7175) (width 0.25) (layer "F.Cu") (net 4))
 (segment (start 91.02 90.85) (end 91.02 89.07) (width 0.25) (layer "F.Cu") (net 4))
 (segment (start 91.847902 91.677902) (end 94.443992 91.677902) (width 0.25) (layer "F.Cu") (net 4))
 (segment (start 94.443992 91.677902) (end 94.461894 91.66) (width 0.25) (layer "F.Cu") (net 4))
 (segment (start 84.2475 82.717966) (end 84.43 82.535466) (width 0.25) (layer "F.Cu") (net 4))
 (segment (start 87.43 68.945) (end 87.105 69.27) (width 0.25) (layer "F.Cu") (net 4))
 (segment (start 84.43 69.36) (end 84.43 70.57) (width 0.25) (layer "F.Cu") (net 4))
 (segment (start 91.847902 91.677902) (end 91.02 90.85) (width 0.25) (layer "F.Cu") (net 4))
 (segment (start 84.2575 85.322034) (end 84.2575 82.727966) (width 0.25) (layer "F.Cu") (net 4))
 (segment (start 91.02 89.07) (end 84.61 89.07) (width 0.25) (layer "F.Cu") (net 4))
 (segment (start 84.43 82.535466) (end 84.43 74.745) (width 0.25) (layer "F.Cu") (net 4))
 (segment (start 85.455 68.345) (end 85.45 68.34) (width 0.25) (layer "F.Cu") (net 4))
 (segment (start 85.405 72.795) (end 85.405 73.3325) (width 0.25) (layer "F.Cu") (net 4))
 (segment (start 84.43 71.82) (end 84.43 70.57) (width 0.25) (layer "F.Cu") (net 4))
 (segment (start 84.2575 88.7175) (end 84.2575 85.322034) (width 0.25) (layer "F.Cu") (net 4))
 (segment (start 85.405 73.3325) (end 84.43 74.3075) (width 0.25) (layer "F.Cu") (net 4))
 (segment (start 87.43 68.345) (end 87.43 68.945) (width 0.25) (layer "F.Cu") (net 4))
 (segment (start 92.3125 85.321568) (end 92.420466 85.429534) (width 0.25) (layer "F.Cu") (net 11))
 (segment (start 93.56 86.74) (end 93.56 89.07) (width 0.25) (layer "F.Cu") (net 11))
 (segment (start 93.56 86.569068) (end 93.56 86.74) (width 0.25) (layer "F.Cu") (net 11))
 (segment (start 92.2725 85.281568) (end 92.420466 85.429534) (width 0.25) (layer "F.Cu") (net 11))
 (segment (start 92.3125 85.321568) (end 92.312034 85.322034) (width 0.25) (layer "F.Cu") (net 11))
 (segment (start 92.2725 74.347788) (end 92.2725 85.281568) (width 0.25) (layer "F.Cu") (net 11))
 (segment (start 87.3825 85.322034) (end 92.312034 85.322034) (width 0.25) (layer "F.Cu") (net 11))
 (segment (start 92.420466 85.429534) (end 93.56 86.569068) (width 0.25) (layer "F.Cu") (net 11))
 (segment (start 86.715 102.31) (end 89.38952 99.63548) (width 0.25) (layer "B.Cu") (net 19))
 (segment (start 89.38952 72.95048) (end 89.83 72.51) (width 0.25) (layer "B.Cu") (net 19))
 (segment (start 89.83 72.51) (end 103.025746 72.51) (width 0.25) (layer "B.Cu") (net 19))
 (segment (start 86.715 104.8475) (end 86.715 102.31) (width 0.25) (layer "B.Cu") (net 19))
 (segment (start 86.7275 104.86) (end 86.715 104.8475) (width 0.25) (layer "B.Cu") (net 19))
 (segment (start 89.38952 99.63548) (end 89.38952 72.95048) (width 0.25) (layer "B.Cu") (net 19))
 (segment (start 94.1875 76.7075) (end 94.1875 74.347788) (width 0.25) (layer "F.Cu") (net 13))
 (segment (start 98.64 78.97) (end 96.45 78.97) (width 0.25) (layer "F.Cu") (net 13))
 (segment (start 98 67.07) (end 102.985746 67.07) (width 0.25) (layer "F.Cu") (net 13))
 (segment (start 102.985746 67.07) (end 103.025746 67.11) (width 0.25) (layer "F.Cu") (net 13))
 (segment (start 94.1875 70.8825) (end 98 67.07) (width 0.25) (layer "F.Cu") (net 13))
 (segment (start 94.1875 74.347788) (end 94.1875 70.8825) (width 0.25) (layer "F.Cu") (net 13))
 (segment (start 96.45 78.97) (end 94.1875 76.7075) (width 0.25) (layer "F.Cu") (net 13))
 (segment (start 96.0125 74.347788) (end 97.6625 74.347788) (width 0.25) (layer "F.Cu") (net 16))
 (segment (start 100.67 91.66) (end 101.18 91.15) (width 0.25) (layer "F.Cu") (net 12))
 (segment (start 101.18 91.15) (end 101.18 89.07) (width 0.25) (layer "F.Cu") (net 12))
 (segment (start 100.74 89.13) (end 101.18 89.57) (width 0.25) (layer "F.Cu") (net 12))
 (segment (start 97.586894 91.66) (end 100.67 91.66) (width 0.25) (layer "F.Cu") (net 12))
 (segment (start 97.0375 102.0925) (end 97.0375 102.985) (width 0.25) (layer "F.Cu") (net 1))
 (segment (start 100.024074 95.196574) (end 100.403426 95.196574) (width 0.25) (layer "F.Cu") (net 1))
 (segment (start 101.064053 102.235947) (end 101.27 102.03) (width 0.25) (layer "F.Cu") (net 1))
 (segment (start 100.4925 102.235947) (end 100.217033 101.96048) (width 0.25) (layer "F.Cu") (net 1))
 (segment (start 101.030947 98.230947) (end 100.4925 98.230947) (width 0.25) (layer "F.Cu") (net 1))
 (segment (start 98.8625 94.035) (end 100.024074 95.196574) (width 0.25) (layer "F.Cu") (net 1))
 (segment (start 97.235 111.839894) (end 97.235 103.1825) (width 0.25) (layer "F.Cu") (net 1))
 (segment (start 101.27 98.47) (end 101.27 95.27) (width 0.25) (layer "F.Cu") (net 1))
 (segment (start 100.217033 101.96048) (end 97.16952 101.96048) (width 0.25) (layer "F.Cu") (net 1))
 (segment (start 100.4925 102.235947) (end 101.064053 102.235947) (width 0.25) (layer "F.Cu") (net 1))
 (segment (start 100.403426 95.196574) (end 101.343426 95.196574) (width 0.25) (layer "F.Cu") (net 1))
 (segment (start 95.86952 101.96048) (end 95.52 102.31) (width 0.25) (layer "F.Cu") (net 1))
 (segment (start 95.52 102.31) (end 94.335 102.31) (width 0.25) (layer "F.Cu") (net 1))
 (segment (start 101.343426 95.196574) (end 103.15104 95.196574) (width 0.25) (layer "F.Cu") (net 1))
 (segment (start 97.16952 101.96048) (end 97.0375 102.0925) (width 0.25) (layer "F.Cu") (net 1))
 (segment (start 101.27 95.27) (end 101.343426 95.196574) (width 0.25) (layer "F.Cu") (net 1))
 (segment (start 97.235 103.1825) (end 97.0375 102.985) (width 0.25) (layer "F.Cu") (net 1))
 (segment (start 101.27 98.47) (end 101.030947 98.230947) (width 0.25) (layer "F.Cu") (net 1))
 (segment (start 101.27 102.03) (end 101.27 98.47) (width 0.25) (layer "F.Cu") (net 1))
 (segment (start 97.16952 101.96048) (end 95.86952 101.96048) (width 0.25) (layer "F.Cu") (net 1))
 (segment (start 103.15104 97.736574) (end 101.75 99.137614) (width 0.25) (layer "F.Cu") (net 17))
 (segment (start 101.565 102.985) (end 98.8625 102.985) (width 0.25) (layer "F.Cu") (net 17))
 (segment (start 101.75 99.137614) (end 101.75 102.8) (width 0.25) (layer "F.Cu") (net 17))
 (segment (start 101.75 102.8) (end 101.565 102.985) (width 0.25) (layer "F.Cu") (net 17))
 (segment (start 94.335 99.77) (end 96.92 99.77) (width 0.25) (layer "F.Cu") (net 14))
 (segment (start 96.92 99.77) (end 97.0375 99.6525) (width 0.25) (layer "F.Cu") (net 14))
 (segment (start 97.0375 99.6525) (end 97.0375 100.7475) (width 0.25) (layer "F.Cu") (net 14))
 (segment (start 97.0375 98.51) (end 97.0375 99.6525) (width 0.25) (layer "F.Cu") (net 14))
 (segment (start 97.381574 102.816574) (end 94.335 99.77) (width 0.25) (layer "B.Cu") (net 14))
 (segment (start 103.15104 102.816574) (end 97.381574 102.816574) (width 0.25) (layer "B.Cu") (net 14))
 (segment (start 87.105 71.87) (end 88.17 71.87) (width 0.25) (layer "F.Cu") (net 10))
 (segment (start 92.11 67.93) (end 92.11 66.84) (width 0.25) (layer "F.Cu") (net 10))
 (segment (start 88.17 71.87) (end 92.11 67.93) (width 0.25) (layer "F.Cu") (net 10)))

